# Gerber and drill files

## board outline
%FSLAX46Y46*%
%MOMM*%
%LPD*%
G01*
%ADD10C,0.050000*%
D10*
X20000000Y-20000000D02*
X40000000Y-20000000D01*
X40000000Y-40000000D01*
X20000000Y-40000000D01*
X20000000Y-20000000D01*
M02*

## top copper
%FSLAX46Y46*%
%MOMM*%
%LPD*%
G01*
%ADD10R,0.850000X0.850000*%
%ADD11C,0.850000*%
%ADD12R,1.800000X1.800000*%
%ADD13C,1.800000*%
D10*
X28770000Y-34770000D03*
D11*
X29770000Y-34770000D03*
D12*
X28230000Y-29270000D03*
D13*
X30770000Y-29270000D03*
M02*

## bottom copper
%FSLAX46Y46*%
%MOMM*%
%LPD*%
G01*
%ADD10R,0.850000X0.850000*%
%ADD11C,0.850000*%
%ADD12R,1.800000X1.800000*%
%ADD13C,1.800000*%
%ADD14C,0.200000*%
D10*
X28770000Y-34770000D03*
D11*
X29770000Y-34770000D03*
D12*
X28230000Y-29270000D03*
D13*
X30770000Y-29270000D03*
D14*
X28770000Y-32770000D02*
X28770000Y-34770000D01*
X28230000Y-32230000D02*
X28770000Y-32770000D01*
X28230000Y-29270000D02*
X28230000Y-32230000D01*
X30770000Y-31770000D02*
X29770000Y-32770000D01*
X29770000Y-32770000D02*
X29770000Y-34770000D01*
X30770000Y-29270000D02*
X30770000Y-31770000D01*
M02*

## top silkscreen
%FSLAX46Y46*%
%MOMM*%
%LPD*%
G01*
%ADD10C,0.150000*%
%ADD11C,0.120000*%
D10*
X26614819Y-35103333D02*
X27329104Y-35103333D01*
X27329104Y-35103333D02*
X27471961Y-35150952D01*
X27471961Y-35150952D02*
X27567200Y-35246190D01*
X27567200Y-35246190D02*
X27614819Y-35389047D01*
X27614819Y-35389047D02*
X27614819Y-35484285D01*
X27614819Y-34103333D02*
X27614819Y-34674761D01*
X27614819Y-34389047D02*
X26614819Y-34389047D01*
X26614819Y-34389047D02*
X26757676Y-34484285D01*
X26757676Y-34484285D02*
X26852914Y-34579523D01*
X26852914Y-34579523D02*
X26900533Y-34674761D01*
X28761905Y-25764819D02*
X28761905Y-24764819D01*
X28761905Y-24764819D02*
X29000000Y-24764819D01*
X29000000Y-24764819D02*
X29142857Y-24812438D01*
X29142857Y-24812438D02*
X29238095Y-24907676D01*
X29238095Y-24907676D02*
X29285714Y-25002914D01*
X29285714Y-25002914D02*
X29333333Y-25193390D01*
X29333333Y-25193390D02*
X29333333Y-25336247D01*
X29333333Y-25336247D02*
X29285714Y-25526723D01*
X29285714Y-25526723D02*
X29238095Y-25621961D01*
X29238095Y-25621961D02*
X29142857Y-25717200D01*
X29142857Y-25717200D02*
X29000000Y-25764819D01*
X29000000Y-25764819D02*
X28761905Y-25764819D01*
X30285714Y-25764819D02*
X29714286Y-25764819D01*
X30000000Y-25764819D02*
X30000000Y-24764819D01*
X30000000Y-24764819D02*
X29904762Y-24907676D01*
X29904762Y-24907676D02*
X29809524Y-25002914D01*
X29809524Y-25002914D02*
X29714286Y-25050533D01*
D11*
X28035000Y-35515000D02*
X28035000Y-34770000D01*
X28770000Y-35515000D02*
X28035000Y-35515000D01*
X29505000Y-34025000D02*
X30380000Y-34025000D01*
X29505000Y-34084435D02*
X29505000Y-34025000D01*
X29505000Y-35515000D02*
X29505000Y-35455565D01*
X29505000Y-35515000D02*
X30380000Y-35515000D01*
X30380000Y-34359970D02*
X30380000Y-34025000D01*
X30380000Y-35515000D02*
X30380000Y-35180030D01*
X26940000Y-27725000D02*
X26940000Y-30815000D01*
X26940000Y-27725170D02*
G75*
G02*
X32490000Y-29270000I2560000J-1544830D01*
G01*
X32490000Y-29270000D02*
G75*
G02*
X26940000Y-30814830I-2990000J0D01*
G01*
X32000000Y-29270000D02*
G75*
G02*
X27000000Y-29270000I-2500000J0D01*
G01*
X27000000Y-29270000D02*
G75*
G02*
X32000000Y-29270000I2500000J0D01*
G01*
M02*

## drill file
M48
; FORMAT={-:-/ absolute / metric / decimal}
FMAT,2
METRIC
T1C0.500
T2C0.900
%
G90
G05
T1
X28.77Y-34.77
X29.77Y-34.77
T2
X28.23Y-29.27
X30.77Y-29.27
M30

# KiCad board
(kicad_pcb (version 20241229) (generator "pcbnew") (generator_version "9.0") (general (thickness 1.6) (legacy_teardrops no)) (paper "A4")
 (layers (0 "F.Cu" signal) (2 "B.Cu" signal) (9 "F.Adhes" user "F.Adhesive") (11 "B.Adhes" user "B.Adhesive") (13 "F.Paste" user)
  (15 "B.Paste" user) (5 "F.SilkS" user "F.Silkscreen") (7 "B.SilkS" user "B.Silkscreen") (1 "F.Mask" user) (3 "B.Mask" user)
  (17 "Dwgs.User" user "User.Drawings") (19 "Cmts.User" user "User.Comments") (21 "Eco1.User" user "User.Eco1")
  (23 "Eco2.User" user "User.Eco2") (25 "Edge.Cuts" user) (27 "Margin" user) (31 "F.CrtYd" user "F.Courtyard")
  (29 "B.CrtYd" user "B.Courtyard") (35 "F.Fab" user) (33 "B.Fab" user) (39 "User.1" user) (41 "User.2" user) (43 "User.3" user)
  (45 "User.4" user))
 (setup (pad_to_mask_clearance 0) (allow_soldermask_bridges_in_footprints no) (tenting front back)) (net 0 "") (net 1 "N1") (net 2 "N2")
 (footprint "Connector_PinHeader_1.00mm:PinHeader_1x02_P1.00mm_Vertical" (layer "F.Cu") (at 28.77 34.77 90)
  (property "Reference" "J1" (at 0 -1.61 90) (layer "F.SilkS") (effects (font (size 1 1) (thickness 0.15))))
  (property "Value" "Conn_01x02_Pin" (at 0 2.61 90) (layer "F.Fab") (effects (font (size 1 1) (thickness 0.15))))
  (fp_line (start -0.745 -0.735) (end 0 -0.735) (stroke (width 0.12) (type solid)) (layer "F.SilkS"))
  (fp_line (start -0.745 0) (end -0.745 -0.735) (stroke (width 0.12) (type solid)) (layer "F.SilkS"))
  (fp_line (start 0.745 0.735) (end 0.745 1.61) (stroke (width 0.12) (type solid)) (layer "F.SilkS"))
  (fp_line (start 0.685565 0.735) (end 0.745 0.735) (stroke (width 0.12) (type solid)) (layer "F.SilkS"))
  (fp_line (start -0.745 0.735) (end -0.685565 0.735) (stroke (width 0.12) (type solid)) (layer "F.SilkS"))
  (fp_line (start -0.745 0.735) (end -0.745 1.61) (stroke (width 0.12) (type solid)) (layer "F.SilkS"))
  (fp_line (start 0.41003 1.61) (end 0.745 1.61) (stroke (width 0.12) (type solid)) (layer "F.SilkS"))
  (fp_line (start -0.745 1.61) (end -0.41003 1.61) (stroke (width 0.12) (type solid)) (layer "F.SilkS"))
  (pad "1" thru_hole rect (at 0 0 90) (size 0.85 0.85) (drill 0.5) (layers "*.Cu" "*.Mask") (remove_unused_layers no) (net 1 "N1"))
  (pad "2" thru_hole circle (at 0 1 90) (size 0.85 0.85) (drill 0.5) (layers "*.Cu" "*.Mask") (remove_unused_layers no) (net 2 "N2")))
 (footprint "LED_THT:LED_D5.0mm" (layer "F.Cu") (at 28.23 29.27)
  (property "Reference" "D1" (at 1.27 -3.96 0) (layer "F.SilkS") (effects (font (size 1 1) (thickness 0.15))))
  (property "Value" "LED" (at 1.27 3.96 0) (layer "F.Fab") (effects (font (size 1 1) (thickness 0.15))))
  (fp_line (start -1.29 -1.545) (end -1.29 1.545) (stroke (width 0.12) (type solid)) (layer "F.SilkS"))
  (fp_arc (start -1.29 -1.54483) (mid 2.071779 -2.880495) (end 4.26 0) (stroke (width 0.12) (type solid)) (layer "F.SilkS"))
  (fp_arc (start 4.26 0) (mid 2.071779 2.880495) (end -1.29 1.54483) (stroke (width 0.12) (type solid)) (layer "F.SilkS"))
  (fp_circle (center 1.27 0) (end 3.77 0) (stroke (width 0.12) (type solid)) (fill no) (layer "F.SilkS"))
  (pad "1" thru_hole rect (at 0 0) (size 1.8 1.8) (drill 0.9) (layers "*.Cu" "*.Mask") (remove_unused_layers no) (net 1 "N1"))
  (pad "2" thru_hole circle (at 2.54 0) (size 1.8 1.8) (drill 0.9) (layers "*.Cu" "*.Mask") (remove_unused_layers no) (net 2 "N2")))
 (gr_rect (start 20 20) (end 40 40) (stroke (width 0.05) (type solid)) (fill no) (layer "Edge.Cuts"))
 (segment (start 28.77 32.77) (end 28.77 34.77) (width 0.2) (layer "B.Cu") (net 1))
 (segment (start 28.23 32.23) (end 28.77 32.77) (width 0.2) (layer "B.Cu") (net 1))
 (segment (start 28.23 29.27) (end 28.23 32.23) (width 0.2) (layer "B.Cu") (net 1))
 (segment (start 30.77 31.77) (end 29.77 32.77) (width 0.2) (layer "B.Cu") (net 2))
 (segment (start 29.77 32.77) (end 29.77 34.77) (width 0.2) (layer "B.Cu") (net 2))
 (segment (start 30.77 29.27) (end 30.77 31.77) (width 0.2) (layer "B.Cu") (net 2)))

